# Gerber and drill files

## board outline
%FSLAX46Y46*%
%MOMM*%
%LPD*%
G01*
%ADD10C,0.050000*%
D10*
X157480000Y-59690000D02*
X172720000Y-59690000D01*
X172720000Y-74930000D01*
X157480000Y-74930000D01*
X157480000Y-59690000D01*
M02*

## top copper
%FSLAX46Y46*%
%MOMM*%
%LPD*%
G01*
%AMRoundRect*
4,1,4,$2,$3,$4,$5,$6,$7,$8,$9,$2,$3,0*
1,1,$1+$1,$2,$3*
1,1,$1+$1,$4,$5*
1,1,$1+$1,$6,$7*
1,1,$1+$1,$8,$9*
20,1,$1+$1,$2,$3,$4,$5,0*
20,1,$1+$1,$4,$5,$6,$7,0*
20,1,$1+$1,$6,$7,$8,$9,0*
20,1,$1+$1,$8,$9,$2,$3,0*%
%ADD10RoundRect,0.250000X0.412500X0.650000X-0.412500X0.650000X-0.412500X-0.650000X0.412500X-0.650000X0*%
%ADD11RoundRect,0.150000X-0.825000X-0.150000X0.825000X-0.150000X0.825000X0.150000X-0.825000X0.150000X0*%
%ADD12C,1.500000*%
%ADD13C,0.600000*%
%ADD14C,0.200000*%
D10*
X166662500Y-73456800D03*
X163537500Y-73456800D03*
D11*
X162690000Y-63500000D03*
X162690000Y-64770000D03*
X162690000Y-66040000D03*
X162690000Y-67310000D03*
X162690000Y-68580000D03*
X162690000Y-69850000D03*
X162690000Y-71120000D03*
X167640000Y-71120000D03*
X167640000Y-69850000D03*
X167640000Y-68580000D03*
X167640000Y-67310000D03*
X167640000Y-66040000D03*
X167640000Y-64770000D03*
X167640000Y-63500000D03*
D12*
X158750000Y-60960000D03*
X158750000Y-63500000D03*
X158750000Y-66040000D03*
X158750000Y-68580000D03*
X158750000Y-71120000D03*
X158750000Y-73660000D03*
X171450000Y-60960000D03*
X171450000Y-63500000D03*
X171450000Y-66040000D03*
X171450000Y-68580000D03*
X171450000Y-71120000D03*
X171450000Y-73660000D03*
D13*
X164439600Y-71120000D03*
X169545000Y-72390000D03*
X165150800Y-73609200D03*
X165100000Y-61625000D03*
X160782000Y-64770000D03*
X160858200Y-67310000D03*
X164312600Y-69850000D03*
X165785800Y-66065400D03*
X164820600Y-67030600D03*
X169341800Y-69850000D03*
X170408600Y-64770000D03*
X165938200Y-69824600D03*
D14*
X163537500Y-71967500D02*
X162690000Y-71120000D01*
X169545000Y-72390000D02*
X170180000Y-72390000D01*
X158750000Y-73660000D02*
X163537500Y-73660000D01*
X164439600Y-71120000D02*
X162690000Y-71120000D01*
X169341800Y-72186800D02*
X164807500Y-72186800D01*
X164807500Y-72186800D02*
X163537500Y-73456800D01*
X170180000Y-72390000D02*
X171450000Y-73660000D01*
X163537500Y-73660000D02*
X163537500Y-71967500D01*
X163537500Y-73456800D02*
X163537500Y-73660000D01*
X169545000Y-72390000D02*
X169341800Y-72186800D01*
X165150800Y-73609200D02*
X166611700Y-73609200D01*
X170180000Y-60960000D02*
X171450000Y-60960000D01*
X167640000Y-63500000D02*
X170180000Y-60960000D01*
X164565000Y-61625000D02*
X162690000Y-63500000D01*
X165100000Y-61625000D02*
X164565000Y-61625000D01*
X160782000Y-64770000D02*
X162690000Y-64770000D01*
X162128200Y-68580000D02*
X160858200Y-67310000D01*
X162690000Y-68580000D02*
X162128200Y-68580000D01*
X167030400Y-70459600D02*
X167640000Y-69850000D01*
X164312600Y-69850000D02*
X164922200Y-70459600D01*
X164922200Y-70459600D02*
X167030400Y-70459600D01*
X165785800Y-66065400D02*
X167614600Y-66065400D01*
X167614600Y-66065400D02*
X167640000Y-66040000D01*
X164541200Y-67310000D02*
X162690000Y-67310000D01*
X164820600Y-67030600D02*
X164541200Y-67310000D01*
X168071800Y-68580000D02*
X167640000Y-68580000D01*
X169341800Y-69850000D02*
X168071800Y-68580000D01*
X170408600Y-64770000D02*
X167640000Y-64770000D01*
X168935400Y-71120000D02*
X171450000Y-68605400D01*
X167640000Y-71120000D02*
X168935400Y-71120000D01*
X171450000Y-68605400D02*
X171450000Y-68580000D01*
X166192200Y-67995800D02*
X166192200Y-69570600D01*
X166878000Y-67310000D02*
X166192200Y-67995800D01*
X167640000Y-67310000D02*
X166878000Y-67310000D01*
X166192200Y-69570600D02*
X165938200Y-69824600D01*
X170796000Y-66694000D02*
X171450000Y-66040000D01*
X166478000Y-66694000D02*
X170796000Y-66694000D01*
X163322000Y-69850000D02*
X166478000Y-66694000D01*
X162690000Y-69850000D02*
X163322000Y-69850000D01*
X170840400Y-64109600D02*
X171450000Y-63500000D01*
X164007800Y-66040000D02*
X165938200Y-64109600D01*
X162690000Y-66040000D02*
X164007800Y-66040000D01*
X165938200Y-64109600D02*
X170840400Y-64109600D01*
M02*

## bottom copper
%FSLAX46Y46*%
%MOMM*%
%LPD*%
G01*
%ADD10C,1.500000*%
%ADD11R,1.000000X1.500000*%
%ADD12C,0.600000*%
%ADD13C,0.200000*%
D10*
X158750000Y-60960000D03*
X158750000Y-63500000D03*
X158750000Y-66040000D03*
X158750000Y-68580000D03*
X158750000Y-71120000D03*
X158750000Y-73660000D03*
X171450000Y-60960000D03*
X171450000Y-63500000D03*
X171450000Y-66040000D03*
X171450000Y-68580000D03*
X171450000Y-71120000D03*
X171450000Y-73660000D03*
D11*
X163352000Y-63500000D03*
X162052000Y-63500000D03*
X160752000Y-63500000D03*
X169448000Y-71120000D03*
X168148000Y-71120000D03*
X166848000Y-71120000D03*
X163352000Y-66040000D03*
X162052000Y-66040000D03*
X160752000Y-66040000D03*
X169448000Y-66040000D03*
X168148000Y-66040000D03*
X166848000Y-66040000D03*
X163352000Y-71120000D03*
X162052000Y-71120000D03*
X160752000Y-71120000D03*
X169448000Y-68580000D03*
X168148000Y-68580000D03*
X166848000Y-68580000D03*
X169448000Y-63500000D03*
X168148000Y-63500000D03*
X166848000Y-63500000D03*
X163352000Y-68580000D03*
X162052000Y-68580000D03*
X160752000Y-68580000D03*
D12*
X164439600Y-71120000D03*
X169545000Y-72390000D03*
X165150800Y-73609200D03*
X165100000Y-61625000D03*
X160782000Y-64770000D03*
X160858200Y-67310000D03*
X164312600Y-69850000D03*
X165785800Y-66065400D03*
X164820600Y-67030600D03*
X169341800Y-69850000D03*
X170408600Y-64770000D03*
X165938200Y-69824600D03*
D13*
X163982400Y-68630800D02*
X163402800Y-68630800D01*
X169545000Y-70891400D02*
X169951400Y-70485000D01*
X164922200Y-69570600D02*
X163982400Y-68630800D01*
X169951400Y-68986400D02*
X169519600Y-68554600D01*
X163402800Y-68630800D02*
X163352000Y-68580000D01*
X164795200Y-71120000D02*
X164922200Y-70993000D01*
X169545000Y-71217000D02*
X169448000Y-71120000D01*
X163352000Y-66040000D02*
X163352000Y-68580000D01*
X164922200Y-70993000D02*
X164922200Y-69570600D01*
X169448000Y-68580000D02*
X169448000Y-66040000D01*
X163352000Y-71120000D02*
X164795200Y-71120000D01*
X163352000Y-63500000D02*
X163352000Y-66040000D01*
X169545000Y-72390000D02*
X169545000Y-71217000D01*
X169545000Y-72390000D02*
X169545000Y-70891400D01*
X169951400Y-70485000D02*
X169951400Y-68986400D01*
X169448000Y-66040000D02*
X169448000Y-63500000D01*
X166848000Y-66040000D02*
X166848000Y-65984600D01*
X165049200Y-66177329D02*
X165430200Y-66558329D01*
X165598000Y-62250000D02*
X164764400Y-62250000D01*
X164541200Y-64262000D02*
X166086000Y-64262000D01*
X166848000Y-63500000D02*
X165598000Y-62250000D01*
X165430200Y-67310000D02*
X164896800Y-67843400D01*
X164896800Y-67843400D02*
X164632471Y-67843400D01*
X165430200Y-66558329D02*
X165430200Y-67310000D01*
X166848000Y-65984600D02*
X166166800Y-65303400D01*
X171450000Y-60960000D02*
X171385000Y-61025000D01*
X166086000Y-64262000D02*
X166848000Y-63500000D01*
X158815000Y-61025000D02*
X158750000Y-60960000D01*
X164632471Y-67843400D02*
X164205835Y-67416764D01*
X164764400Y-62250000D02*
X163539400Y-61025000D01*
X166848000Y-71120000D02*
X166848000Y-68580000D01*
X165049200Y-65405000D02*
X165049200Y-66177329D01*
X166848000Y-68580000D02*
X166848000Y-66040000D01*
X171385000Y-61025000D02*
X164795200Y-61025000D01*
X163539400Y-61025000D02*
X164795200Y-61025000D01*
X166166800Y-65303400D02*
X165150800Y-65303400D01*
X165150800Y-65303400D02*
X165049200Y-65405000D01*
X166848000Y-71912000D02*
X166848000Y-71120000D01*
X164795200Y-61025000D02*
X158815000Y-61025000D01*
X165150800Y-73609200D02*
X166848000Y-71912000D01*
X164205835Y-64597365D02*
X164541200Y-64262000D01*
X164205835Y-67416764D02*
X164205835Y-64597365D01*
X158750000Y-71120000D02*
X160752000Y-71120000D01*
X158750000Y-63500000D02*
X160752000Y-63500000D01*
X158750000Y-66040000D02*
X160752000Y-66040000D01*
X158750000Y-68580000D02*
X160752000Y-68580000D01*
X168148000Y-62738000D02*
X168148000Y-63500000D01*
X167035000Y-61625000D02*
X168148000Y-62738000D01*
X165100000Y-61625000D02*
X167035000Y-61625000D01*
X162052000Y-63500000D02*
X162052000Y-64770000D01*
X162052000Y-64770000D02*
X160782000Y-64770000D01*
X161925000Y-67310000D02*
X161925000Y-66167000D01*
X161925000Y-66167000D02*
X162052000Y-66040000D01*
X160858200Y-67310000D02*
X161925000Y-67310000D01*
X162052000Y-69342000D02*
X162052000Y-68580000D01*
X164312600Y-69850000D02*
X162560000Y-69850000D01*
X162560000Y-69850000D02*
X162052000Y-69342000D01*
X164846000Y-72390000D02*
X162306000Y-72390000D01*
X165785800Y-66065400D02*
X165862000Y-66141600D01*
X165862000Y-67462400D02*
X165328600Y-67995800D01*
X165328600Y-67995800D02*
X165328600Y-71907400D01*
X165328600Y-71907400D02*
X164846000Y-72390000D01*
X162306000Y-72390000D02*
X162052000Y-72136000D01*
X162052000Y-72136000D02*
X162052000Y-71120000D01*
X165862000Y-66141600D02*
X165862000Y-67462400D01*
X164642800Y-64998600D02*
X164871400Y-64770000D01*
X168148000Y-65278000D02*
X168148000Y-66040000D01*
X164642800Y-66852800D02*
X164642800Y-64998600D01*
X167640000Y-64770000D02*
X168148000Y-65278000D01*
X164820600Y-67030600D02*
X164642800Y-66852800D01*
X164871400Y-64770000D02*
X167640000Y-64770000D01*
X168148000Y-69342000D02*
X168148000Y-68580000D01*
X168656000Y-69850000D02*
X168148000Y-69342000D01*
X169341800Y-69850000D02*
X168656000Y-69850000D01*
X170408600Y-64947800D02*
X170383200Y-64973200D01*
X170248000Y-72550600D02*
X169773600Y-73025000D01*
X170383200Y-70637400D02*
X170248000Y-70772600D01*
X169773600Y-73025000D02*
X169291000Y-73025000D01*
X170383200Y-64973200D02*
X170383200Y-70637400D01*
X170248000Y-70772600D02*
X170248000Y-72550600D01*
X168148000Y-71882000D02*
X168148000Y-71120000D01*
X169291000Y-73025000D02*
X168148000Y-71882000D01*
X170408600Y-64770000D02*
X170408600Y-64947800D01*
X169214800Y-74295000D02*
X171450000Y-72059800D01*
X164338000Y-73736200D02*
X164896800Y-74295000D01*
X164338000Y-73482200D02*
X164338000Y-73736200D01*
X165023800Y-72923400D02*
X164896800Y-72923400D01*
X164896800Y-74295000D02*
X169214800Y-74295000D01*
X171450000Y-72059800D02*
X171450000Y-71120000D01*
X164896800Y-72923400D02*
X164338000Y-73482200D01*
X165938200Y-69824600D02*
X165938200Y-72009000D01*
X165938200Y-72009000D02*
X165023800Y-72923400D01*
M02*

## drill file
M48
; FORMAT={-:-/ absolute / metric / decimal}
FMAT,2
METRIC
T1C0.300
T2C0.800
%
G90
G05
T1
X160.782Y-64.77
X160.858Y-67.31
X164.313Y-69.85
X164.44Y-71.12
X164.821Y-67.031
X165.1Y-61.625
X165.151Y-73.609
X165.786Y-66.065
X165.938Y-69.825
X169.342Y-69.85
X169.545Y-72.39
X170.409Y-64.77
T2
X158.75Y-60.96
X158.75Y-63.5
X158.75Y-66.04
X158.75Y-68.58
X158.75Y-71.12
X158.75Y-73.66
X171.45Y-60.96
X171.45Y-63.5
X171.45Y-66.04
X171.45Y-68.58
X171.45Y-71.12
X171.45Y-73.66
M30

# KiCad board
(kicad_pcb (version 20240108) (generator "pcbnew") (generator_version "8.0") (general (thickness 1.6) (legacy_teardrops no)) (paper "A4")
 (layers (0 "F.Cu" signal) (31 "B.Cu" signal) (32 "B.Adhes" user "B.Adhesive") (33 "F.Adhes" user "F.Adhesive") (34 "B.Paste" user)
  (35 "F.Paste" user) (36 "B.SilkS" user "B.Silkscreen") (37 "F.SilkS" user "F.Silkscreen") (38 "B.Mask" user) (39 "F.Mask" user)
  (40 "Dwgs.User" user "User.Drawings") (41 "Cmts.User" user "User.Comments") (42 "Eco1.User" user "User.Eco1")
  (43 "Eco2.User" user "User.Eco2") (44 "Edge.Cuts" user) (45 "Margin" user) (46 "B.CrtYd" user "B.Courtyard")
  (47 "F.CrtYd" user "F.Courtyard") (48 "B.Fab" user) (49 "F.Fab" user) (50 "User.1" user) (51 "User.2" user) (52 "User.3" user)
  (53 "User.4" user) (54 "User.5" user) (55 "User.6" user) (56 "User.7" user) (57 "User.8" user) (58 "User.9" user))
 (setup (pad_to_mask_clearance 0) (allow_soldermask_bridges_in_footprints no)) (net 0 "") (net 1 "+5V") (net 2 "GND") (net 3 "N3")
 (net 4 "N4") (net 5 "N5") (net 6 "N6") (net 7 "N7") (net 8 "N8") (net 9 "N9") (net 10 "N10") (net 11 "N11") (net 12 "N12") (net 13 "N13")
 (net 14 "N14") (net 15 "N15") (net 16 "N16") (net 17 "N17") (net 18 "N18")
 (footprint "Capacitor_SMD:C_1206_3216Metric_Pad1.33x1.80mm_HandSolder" (layer "F.Cu") (at 165.1 73.4568 180)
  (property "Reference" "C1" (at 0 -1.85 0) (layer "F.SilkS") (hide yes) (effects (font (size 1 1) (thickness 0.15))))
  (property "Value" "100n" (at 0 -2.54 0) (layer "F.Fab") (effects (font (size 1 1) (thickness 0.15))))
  (pad "1" smd roundrect (at -1.5625 0 180) (size 1.325 1.8) (layers "F.Cu" "F.Paste" "F.Mask") (roundrect_rratio 0.188679) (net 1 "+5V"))
  (pad "2" smd roundrect (at 1.5625 0 180) (size 1.325 1.8) (layers "F.Cu" "F.Paste" "F.Mask") (roundrect_rratio 0.188679) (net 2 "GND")))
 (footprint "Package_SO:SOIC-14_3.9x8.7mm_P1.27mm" (layer "F.Cu") (at 165.165 67.31)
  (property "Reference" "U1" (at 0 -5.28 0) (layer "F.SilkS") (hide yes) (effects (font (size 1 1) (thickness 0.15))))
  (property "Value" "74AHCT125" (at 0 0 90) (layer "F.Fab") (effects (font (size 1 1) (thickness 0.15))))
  (pad "1" smd roundrect (at -2.475 -3.81) (size 1.95 0.6) (layers "F.Cu" "F.Paste" "F.Mask") (roundrect_rratio 0.25) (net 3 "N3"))
  (pad "2" smd roundrect (at -2.475 -2.54) (size 1.95 0.6) (layers "F.Cu" "F.Paste" "F.Mask") (roundrect_rratio 0.25) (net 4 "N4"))
  (pad "3" smd roundrect (at -2.475 -1.27) (size 1.95 0.6) (layers "F.Cu" "F.Paste" "F.Mask") (roundrect_rratio 0.25) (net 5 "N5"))
  (pad "4" smd roundrect (at -2.475 0) (size 1.95 0.6) (layers "F.Cu" "F.Paste" "F.Mask") (roundrect_rratio 0.25) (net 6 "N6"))
  (pad "5" smd roundrect (at -2.475 1.27) (size 1.95 0.6) (layers "F.Cu" "F.Paste" "F.Mask") (roundrect_rratio 0.25) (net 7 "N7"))
  (pad "6" smd roundrect (at -2.475 2.54) (size 1.95 0.6) (layers "F.Cu" "F.Paste" "F.Mask") (roundrect_rratio 0.25) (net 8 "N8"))
  (pad "7" smd roundrect (at -2.475 3.81) (size 1.95 0.6) (layers "F.Cu" "F.Paste" "F.Mask") (roundrect_rratio 0.25) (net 2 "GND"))
  (pad "8" smd roundrect (at 2.475 3.81) (size 1.95 0.6) (layers "F.Cu" "F.Paste" "F.Mask") (roundrect_rratio 0.25) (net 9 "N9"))
  (pad "9" smd roundrect (at 2.475 2.54) (size 1.95 0.6) (layers "F.Cu" "F.Paste" "F.Mask") (roundrect_rratio 0.25) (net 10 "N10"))
  (pad "10" smd roundrect (at 2.475 1.27) (size 1.95 0.6) (layers "F.Cu" "F.Paste" "F.Mask") (roundrect_rratio 0.25) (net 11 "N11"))
  (pad "11" smd roundrect (at 2.475 0) (size 1.95 0.6) (layers "F.Cu" "F.Paste" "F.Mask") (roundrect_rratio 0.25) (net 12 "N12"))
  (pad "12" smd roundrect (at 2.475 -1.27) (size 1.95 0.6) (layers "F.Cu" "F.Paste" "F.Mask") (roundrect_rratio 0.25) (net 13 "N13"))
  (pad "13" smd roundrect (at 2.475 -2.54) (size 1.95 0.6) (layers "F.Cu" "F.Paste" "F.Mask") (roundrect_rratio 0.25) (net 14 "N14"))
  (pad "14" smd roundrect (at 2.475 -3.81) (size 1.95 0.6) (layers "F.Cu" "F.Paste" "F.Mask") (roundrect_rratio 0.25) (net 1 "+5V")))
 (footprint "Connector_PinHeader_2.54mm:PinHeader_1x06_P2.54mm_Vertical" (layer "F.Cu") (at 158.75 60.96)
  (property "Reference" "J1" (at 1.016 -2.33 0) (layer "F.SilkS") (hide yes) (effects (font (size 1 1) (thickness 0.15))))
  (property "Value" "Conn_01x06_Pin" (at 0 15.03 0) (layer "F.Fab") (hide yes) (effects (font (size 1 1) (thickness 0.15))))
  (pad "1" thru_hole circle (at 0 0) (size 1.5 1.5) (drill 0.8) (layers "*.Cu" "*.Mask") (remove_unused_layers no) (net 1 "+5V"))
  (pad "2" thru_hole circle (at 0 2.54) (size 1.5 1.5) (drill 0.8) (layers "*.Cu" "*.Mask") (remove_unused_layers no) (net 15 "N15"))
  (pad "3" thru_hole circle (at 0 5.08) (size 1.5 1.5) (drill 0.8) (layers "*.Cu" "*.Mask") (remove_unused_layers no) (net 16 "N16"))
  (pad "4" thru_hole circle (at 0 7.62) (size 1.5 1.5) (drill 0.8) (layers "*.Cu" "*.Mask") (remove_unused_layers no) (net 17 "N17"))
  (pad "5" thru_hole circle (at 0 10.16) (size 1.5 1.5) (drill 0.8) (layers "*.Cu" "*.Mask") (remove_unused_layers no) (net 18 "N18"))
  (pad "6" thru_hole circle (at 0 12.7) (size 1.5 1.5) (drill 0.8) (layers "*.Cu" "*.Mask") (remove_unused_layers no) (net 2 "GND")))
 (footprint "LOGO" (layer "F.Cu") (at 165.09997 60.628602)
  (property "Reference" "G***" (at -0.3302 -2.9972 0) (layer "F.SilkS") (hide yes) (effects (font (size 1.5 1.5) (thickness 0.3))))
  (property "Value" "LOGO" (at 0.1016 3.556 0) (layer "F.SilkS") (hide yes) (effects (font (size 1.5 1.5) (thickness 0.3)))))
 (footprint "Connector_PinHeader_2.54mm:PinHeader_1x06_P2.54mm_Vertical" (layer "F.Cu") (at 171.45 60.96)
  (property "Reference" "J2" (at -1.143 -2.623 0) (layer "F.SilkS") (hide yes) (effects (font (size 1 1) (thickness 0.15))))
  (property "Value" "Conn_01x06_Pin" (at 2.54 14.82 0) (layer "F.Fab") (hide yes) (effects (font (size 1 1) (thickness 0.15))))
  (pad "1" thru_hole circle (at 0 0 180) (size 1.5 1.5) (drill 0.8) (layers "*.Cu" "*.Mask") (remove_unused_layers no) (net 1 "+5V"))
  (pad "2" thru_hole circle (at 0 2.54 180) (size 1.5 1.5) (drill 0.8) (layers "*.Cu" "*.Mask") (remove_unused_layers no) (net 5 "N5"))
  (pad "3" thru_hole circle (at 0 5.08 180) (size 1.5 1.5) (drill 0.8) (layers "*.Cu" "*.Mask") (remove_unused_layers no) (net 8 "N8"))
  (pad "4" thru_hole circle (at 0 7.62 180) (size 1.5 1.5) (drill 0.8) (layers "*.Cu" "*.Mask") (remove_unused_layers no) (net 9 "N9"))
  (pad "5" thru_hole circle (at 0 10.16 180) (size 1.5 1.5) (drill 0.8) (layers "*.Cu" "*.Mask") (remove_unused_layers no) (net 12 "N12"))
  (pad "6" thru_hole circle (at 0 12.7 180) (size 1.5 1.5) (drill 0.8) (layers "*.Cu" "*.Mask") (remove_unused_layers no) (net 2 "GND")))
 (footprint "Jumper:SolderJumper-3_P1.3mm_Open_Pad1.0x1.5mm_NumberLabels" (layer "B.Cu") (at 162.052 63.5 180)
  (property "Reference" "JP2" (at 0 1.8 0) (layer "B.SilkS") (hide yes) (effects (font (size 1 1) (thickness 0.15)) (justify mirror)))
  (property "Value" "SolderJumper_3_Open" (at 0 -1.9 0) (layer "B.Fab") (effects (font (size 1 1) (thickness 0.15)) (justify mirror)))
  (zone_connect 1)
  (pad "1" smd rect (at -1.3 0 180) (size 1 1.5) (layers "B.Cu" "B.Mask") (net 2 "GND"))
  (pad "2" smd rect (at 0 0 180) (size 1 1.5) (layers "B.Cu" "B.Mask") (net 4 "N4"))
  (pad "3" smd rect (at 1.3 0 180) (size 1 1.5) (layers "B.Cu" "B.Mask") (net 15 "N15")))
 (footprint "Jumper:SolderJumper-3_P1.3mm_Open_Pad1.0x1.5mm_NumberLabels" (layer "B.Cu") (at 168.148 71.12 180)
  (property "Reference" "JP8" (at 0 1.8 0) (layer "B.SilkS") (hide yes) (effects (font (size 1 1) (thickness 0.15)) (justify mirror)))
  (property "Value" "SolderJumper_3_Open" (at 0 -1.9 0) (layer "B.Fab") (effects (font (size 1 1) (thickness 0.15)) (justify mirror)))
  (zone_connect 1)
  (pad "1" smd rect (at -1.3 0 180) (size 1 1.5) (layers "B.Cu" "B.Mask") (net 2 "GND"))
  (pad "2" smd rect (at 0 0 180) (size 1 1.5) (layers "B.Cu" "B.Mask") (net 14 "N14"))
  (pad "3" smd rect (at 1.3 0 180) (size 1 1.5) (layers "B.Cu" "B.Mask") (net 1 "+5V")))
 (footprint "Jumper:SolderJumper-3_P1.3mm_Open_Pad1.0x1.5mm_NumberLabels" (layer "B.Cu") (at 162.052 66.04 180)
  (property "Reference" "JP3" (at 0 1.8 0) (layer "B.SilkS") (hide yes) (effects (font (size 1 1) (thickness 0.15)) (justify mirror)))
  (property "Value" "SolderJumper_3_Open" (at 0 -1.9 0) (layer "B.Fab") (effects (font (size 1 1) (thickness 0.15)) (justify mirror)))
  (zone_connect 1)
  (pad "1" smd rect (at -1.3 0 180) (size 1 1.5) (layers "B.Cu" "B.Mask") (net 2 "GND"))
  (pad "2" smd rect (at 0 0 180) (size 1 1.5) (layers "B.Cu" "B.Mask") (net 7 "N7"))
  (pad "3" smd rect (at 1.3 0 180) (size 1 1.5) (layers "B.Cu" "B.Mask") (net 16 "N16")))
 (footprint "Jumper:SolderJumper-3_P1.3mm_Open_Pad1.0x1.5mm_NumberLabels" (layer "B.Cu") (at 168.148 66.04 180)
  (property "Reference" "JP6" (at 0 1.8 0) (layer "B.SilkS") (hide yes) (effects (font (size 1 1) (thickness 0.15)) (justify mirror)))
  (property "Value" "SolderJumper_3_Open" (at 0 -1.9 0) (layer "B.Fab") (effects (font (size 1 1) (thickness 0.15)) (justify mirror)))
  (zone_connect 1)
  (pad "1" smd rect (at -1.3 0 180) (size 1 1.5) (layers "B.Cu" "B.Mask") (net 2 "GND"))
  (pad "2" smd rect (at 0 0 180) (size 1 1.5) (layers "B.Cu" "B.Mask") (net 6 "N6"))
  (pad "3" smd rect (at 1.3 0 180) (size 1 1.5) (layers "B.Cu" "B.Mask") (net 1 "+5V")))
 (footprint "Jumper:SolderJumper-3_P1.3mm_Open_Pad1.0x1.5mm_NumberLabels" (layer "B.Cu") (at 162.052 71.12 180)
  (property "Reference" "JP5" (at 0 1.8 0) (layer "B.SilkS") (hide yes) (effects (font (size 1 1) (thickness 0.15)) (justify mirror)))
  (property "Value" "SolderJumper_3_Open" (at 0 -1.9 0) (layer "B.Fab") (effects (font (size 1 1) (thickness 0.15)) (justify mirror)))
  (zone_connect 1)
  (pad "1" smd rect (at -1.3 0 180) (size 1 1.5) (layers "B.Cu" "B.Mask") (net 2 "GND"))
  (pad "2" smd rect (at 0 0 180) (size 1 1.5) (layers "B.Cu" "B.Mask") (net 13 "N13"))
  (pad "3" smd rect (at 1.3 0 180) (size 1 1.5) (layers "B.Cu" "B.Mask") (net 18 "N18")))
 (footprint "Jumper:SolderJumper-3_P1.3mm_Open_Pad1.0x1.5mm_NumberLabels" (layer "B.Cu") (at 168.148 68.58 180)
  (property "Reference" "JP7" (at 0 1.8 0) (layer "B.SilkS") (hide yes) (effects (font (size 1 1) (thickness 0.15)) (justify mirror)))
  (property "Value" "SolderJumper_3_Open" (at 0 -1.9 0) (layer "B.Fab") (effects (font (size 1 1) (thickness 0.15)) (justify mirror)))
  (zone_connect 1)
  (pad "1" smd rect (at -1.3 0 180) (size 1 1.5) (layers "B.Cu" "B.Mask") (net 2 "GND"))
  (pad "2" smd rect (at 0 0 180) (size 1 1.5) (layers "B.Cu" "B.Mask") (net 11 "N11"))
  (pad "3" smd rect (at 1.3 0 180) (size 1 1.5) (layers "B.Cu" "B.Mask") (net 1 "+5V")))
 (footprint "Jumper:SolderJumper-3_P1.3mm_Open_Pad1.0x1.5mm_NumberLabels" (layer "B.Cu") (at 168.148 63.5 180)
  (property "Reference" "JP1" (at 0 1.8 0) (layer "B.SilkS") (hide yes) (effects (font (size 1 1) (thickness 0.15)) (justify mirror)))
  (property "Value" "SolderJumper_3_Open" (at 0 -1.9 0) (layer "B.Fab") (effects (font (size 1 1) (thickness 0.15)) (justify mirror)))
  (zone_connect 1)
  (pad "1" smd rect (at -1.3 0 180) (size 1 1.5) (layers "B.Cu" "B.Mask") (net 2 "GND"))
  (pad "2" smd rect (at 0 0 180) (size 1 1.5) (layers "B.Cu" "B.Mask") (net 3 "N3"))
  (pad "3" smd rect (at 1.3 0 180) (size 1 1.5) (layers "B.Cu" "B.Mask") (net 1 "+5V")))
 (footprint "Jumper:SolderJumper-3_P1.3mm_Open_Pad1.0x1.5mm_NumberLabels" (layer "B.Cu") (at 162.052 68.58 180)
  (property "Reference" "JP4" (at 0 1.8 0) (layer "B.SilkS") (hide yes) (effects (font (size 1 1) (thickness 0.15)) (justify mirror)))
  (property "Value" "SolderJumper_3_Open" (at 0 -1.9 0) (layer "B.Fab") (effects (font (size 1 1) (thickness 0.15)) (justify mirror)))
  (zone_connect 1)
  (pad "1" smd rect (at -1.3 0 180) (size 1 1.5) (layers "B.Cu" "B.Mask") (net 2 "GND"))
  (pad "2" smd rect (at 0 0 180) (size 1 1.5) (layers "B.Cu" "B.Mask") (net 10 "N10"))
  (pad "3" smd rect (at 1.3 0 180) (size 1 1.5) (layers "B.Cu" "B.Mask") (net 17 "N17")))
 (gr_rect (start 157.48 59.69) (end 172.72 74.93) (locked yes) (stroke (width 0.05) (type default)) (fill none) (layer "Edge.Cuts"))
 (segment (start 163.5375 71.9675) (end 162.69 71.12) (width 0.2) (layer "F.Cu") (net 2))
 (segment (start 169.545 72.39) (end 170.18 72.39) (width 0.2) (layer "F.Cu") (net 2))
 (segment (start 158.75 73.66) (end 163.5375 73.66) (width 0.2) (layer "F.Cu") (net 2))
 (segment (start 164.4396 71.12) (end 162.69 71.12) (width 0.2) (layer "F.Cu") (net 2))
 (segment (start 169.3418 72.1868) (end 164.8075 72.1868) (width 0.2) (layer "F.Cu") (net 2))
 (segment (start 164.8075 72.1868) (end 163.5375 73.4568) (width 0.2) (layer "F.Cu") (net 2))
 (segment (start 170.18 72.39) (end 171.45 73.66) (width 0.2) (layer "F.Cu") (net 2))
 (segment (start 163.5375 73.66) (end 163.5375 71.9675) (width 0.2) (layer "F.Cu") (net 2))
 (segment (start 163.5375 73.4568) (end 163.5375 73.66) (width 0.2) (layer "F.Cu") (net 2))
 (segment (start 169.545 72.39) (end 169.3418 72.1868) (width 0.2) (layer "F.Cu") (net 2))
 (via (at 164.4396 71.12) (size 0.6) (drill 0.3) (layers "F.Cu" "B.Cu") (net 2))
 (via (at 169.545 72.39) (size 0.6) (drill 0.3) (layers "F.Cu" "B.Cu") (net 2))
 (segment (start 163.9824 68.6308) (end 163.4028 68.6308) (width 0.2) (layer "B.Cu") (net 2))
 (segment (start 169.545 70.8914) (end 169.9514 70.485) (width 0.2) (layer "B.Cu") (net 2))
 (segment (start 164.9222 69.5706) (end 163.9824 68.6308) (width 0.2) (layer "B.Cu") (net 2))
 (segment (start 169.9514 68.9864) (end 169.5196 68.5546) (width 0.2) (layer "B.Cu") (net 2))
 (segment (start 163.4028 68.6308) (end 163.352 68.58) (width 0.2) (layer "B.Cu") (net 2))
 (segment (start 164.7952 71.12) (end 164.9222 70.993) (width 0.2) (layer "B.Cu") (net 2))
 (segment (start 169.545 71.217) (end 169.448 71.12) (width 0.2) (layer "B.Cu") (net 2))
 (segment (start 163.352 66.04) (end 163.352 68.58) (width 0.2) (layer "B.Cu") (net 2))
 (segment (start 164.9222 70.993) (end 164.9222 69.5706) (width 0.2) (layer "B.Cu") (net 2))
 (segment (start 169.448 68.58) (end 169.448 66.04) (width 0.2) (layer "B.Cu") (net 2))
 (segment (start 163.352 71.12) (end 164.7952 71.12) (width 0.2) (layer "B.Cu") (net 2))
 (segment (start 163.352 63.5) (end 163.352 66.04) (width 0.2) (layer "B.Cu") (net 2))
 (segment (start 169.545 72.39) (end 169.545 71.217) (width 0.2) (layer "B.Cu") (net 2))
 (segment (start 169.545 72.39) (end 169.545 70.8914) (width 0.2) (layer "B.Cu") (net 2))
 (segment (start 169.9514 70.485) (end 169.9514 68.9864) (width 0.2) (layer "B.Cu") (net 2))
 (segment (start 169.448 66.04) (end 169.448 63.5) (width 0.2) (layer "B.Cu") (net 2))
 (segment (start 165.1508 73.6092) (end 166.6117 73.6092) (width 0.2) (layer "F.Cu") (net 1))
 (segment (start 170.18 60.96) (end 171.45 60.96) (width 0.2) (layer "F.Cu") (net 1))
 (segment (start 167.64 63.5) (end 170.18 60.96) (width 0.2) (layer "F.Cu") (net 1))
 (via (at 165.1508 73.6092) (size 0.6) (drill 0.3) (layers "F.Cu" "B.Cu") (free yes) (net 1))
 (segment (start 166.848 66.04) (end 166.848 65.9846) (width 0.2) (layer "B.Cu") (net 1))
 (segment (start 165.0492 66.177329) (end 165.4302 66.558329) (width 0.2) (layer "B.Cu") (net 1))
 (segment (start 165.598 62.25) (end 164.7644 62.25) (width 0.2) (layer "B.Cu") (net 1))
 (segment (start 164.5412 64.262) (end 166.086 64.262) (width 0.2) (layer "B.Cu") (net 1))
 (segment (start 166.848 63.5) (end 165.598 62.25) (width 0.2) (layer "B.Cu") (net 1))
 (segment (start 165.4302 67.31) (end 164.8968 67.8434) (width 0.2) (layer "B.Cu") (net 1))
 (segment (start 164.8968 67.8434) (end 164.632471 67.8434) (width 0.2) (layer "B.Cu") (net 1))
 (segment (start 165.4302 66.558329) (end 165.4302 67.31) (width 0.2) (layer "B.Cu") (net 1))
 (segment (start 166.848 65.9846) (end 166.1668 65.3034) (width 0.2) (layer "B.Cu") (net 1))
 (segment (start 171.45 60.96) (end 171.385 61.025) (width 0.2) (layer "B.Cu") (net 1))
 (segment (start 166.086 64.262) (end 166.848 63.5) (width 0.2) (layer "B.Cu") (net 1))
 (segment (start 158.815 61.025) (end 158.75 60.96) (width 0.2) (layer "B.Cu") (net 1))
 (segment (start 164.632471 67.8434) (end 164.205835 67.416764) (width 0.2) (layer "B.Cu") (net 1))
 (segment (start 164.7644 62.25) (end 163.5394 61.025) (width 0.2) (layer "B.Cu") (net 1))
 (segment (start 166.848 71.12) (end 166.848 68.58) (width 0.2) (layer "B.Cu") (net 1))
 (segment (start 165.0492 65.405) (end 165.0492 66.177329) (width 0.2) (layer "B.Cu") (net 1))
 (segment (start 166.848 68.58) (end 166.848 66.04) (width 0.2) (layer "B.Cu") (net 1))
 (segment (start 171.385 61.025) (end 164.7952 61.025) (width 0.2) (layer "B.Cu") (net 1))
 (segment (start 163.5394 61.025) (end 164.7952 61.025) (width 0.2) (layer "B.Cu") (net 1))
 (segment (start 166.1668 65.3034) (end 165.1508 65.3034) (width 0.2) (layer "B.Cu") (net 1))
 (segment (start 165.1508 65.3034) (end 165.0492 65.405) (width 0.2) (layer "B.Cu") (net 1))
 (segment (start 166.848 71.912) (end 166.848 71.12) (width 0.2) (layer "B.Cu") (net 1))
 (segment (start 164.7952 61.025) (end 158.815 61.025) (width 0.2) (layer "B.Cu") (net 1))
 (segment (start 165.1508 73.6092) (end 166.848 71.912) (width 0.2) (layer "B.Cu") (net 1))
 (segment (start 164.205835 64.597365) (end 164.5412 64.262) (width 0.2) (layer "B.Cu") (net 1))
 (segment (start 164.205835 67.416764) (end 164.205835 64.597365) (width 0.2) (layer "B.Cu") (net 1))
 (segment (start 158.75 71.12) (end 160.752 71.12) (width 0.2) (layer "B.Cu") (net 18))
 (segment (start 158.75 63.5) (end 160.752 63.5) (width 0.2) (layer "B.Cu") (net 15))
 (segment (start 158.75 66.04) (end 160.752 66.04) (width 0.2) (layer "B.Cu") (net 16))
 (segment (start 158.75 68.58) (end 160.752 68.58) (width 0.2) (layer "B.Cu") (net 17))
 (segment (start 164.565 61.625) (end 162.69 63.5) (width 0.2) (layer "F.Cu") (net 3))
 (segment (start 165.1 61.625) (end 164.565 61.625) (width 0.2) (layer "F.Cu") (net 3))
 (via (at 165.1 61.625) (size 0.6) (drill 0.3) (layers "F.Cu" "B.Cu") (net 3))
 (segment (start 168.148 62.738) (end 168.148 63.5) (width 0.2) (layer "B.Cu") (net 3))
 (segment (start 167.035 61.625) (end 168.148 62.738) (width 0.2) (layer "B.Cu") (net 3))
 (segment (start 165.1 61.625) (end 167.035 61.625) (width 0.2) (layer "B.Cu") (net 3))
 (segment (start 160.782 64.77) (end 162.69 64.77) (width 0.2) (layer "F.Cu") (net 4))
 (via (at 160.782 64.77) (size 0.6) (drill 0.3) (layers "F.Cu" "B.Cu") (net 4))
 (segment (start 162.052 63.5) (end 162.052 64.77) (width 0.2) (layer "B.Cu") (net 4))
 (segment (start 162.052 64.77) (end 160.782 64.77) (width 0.2) (layer "B.Cu") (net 4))
 (segment (start 162.1282 68.58) (end 160.8582 67.31) (width 0.2) (layer "F.Cu") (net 7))
 (segment (start 162.69 68.58) (end 162.1282 68.58) (width 0.2) (layer "F.Cu") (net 7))
 (via (at 160.8582 67.31) (size 0.6) (drill 0.3) (layers "F.Cu" "B.Cu") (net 7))
 (segment (start 161.925 67.31) (end 161.925 66.167) (width 0.2) (layer "B.Cu") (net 7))
 (segment (start 161.925 66.167) (end 162.052 66.04) (width 0.2) (layer "B.Cu") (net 7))
 (segment (start 160.8582 67.31) (end 161.925 67.31) (width 0.2) (layer "B.Cu") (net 7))
 (segment (start 167.0304 70.4596) (end 167.64 69.85) (width 0.2) (layer "F.Cu") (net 10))
 (segment (start 164.3126 69.85) (end 164.9222 70.4596) (width 0.2) (layer "F.Cu") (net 10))
 (segment (start 164.9222 70.4596) (end 167.0304 70.4596) (width 0.2) (layer "F.Cu") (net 10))
 (via (at 164.3126 69.85) (size 0.6) (drill 0.3) (layers "F.Cu" "B.Cu") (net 10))
 (segment (start 162.052 69.342) (end 162.052 68.58) (width 0.2) (layer "B.Cu") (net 10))
 (segment (start 164.3126 69.85) (end 162.56 69.85) (width 0.2) (layer "B.Cu") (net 10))
 (segment (start 162.56 69.85) (end 162.052 69.342) (width 0.2) (layer "B.Cu") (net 10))
 (segment (start 165.7858 66.0654) (end 167.6146 66.0654) (width 0.2) (layer "F.Cu") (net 13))
 (segment (start 167.6146 66.0654) (end 167.64 66.04) (width 0.2) (layer "F.Cu") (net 13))
 (via (at 165.7858 66.0654) (size 0.6) (drill 0.3) (layers "F.Cu" "B.Cu") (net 13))
 (segment (start 164.846 72.39) (end 162.306 72.39) (width 0.2) (layer "B.Cu") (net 13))
 (segment (start 165.7858 66.0654) (end 165.862 66.1416) (width 0.2) (layer "B.Cu") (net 13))
 (segment (start 165.862 67.4624) (end 165.3286 67.9958) (width 0.2) (layer "B.Cu") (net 13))
 (segment (start 165.3286 67.9958) (end 165.3286 71.9074) (width 0.2) (layer "B.Cu") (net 13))
 (segment (start 165.3286 71.9074) (end 164.846 72.39) (width 0.2) (layer "B.Cu") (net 13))
 (segment (start 162.306 72.39) (end 162.052 72.136) (width 0.2) (layer "B.Cu") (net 13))
 (segment (start 162.052 72.136) (end 162.052 71.12) (width 0.2) (layer "B.Cu") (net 13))
 (segment (start 165.862 66.1416) (end 165.862 67.4624) (width 0.2) (layer "B.Cu") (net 13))
 (segment (start 164.5412 67.31) (end 162.69 67.31) (width 0.2) (layer "F.Cu") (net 6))
 (segment (start 164.8206 67.0306) (end 164.5412 67.31) (width 0.2) (layer "F.Cu") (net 6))
 (via (at 164.8206 67.0306) (size 0.6) (drill 0.3) (layers "F.Cu" "B.Cu") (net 6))
 (segment (start 164.6428 64.9986) (end 164.8714 64.77) (width 0.2) (layer "B.Cu") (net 6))
 (segment (start 168.148 65.278) (end 168.148 66.04) (width 0.2) (layer "B.Cu") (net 6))
 (segment (start 164.6428 66.8528) (end 164.6428 64.9986) (width 0.2) (layer "B.Cu") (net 6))
 (segment (start 167.64 64.77) (end 168.148 65.278) (width 0.2) (layer "B.Cu") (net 6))
 (segment (start 164.8206 67.0306) (end 164.6428 66.8528) (width 0.2) (layer "B.Cu") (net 6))
 (segment (start 164.8714 64.77) (end 167.64 64.77) (width 0.2) (layer "B.Cu") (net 6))
 (segment (start 168.0718 68.58) (end 167.64 68.58) (width 0.2) (layer "F.Cu") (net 11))
 (segment (start 169.3418 69.85) (end 168.0718 68.58) (width 0.2) (layer "F.Cu") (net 11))
 (via (at 169.3418 69.85) (size 0.6) (drill 0.3) (layers "F.Cu" "B.Cu") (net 11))
 (segment (start 168.148 69.342) (end 168.148 68.58) (width 0.2) (layer "B.Cu") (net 11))
 (segment (start 168.656 69.85) (end 168.148 69.342) (width 0.2) (layer "B.Cu") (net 11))
 (segment (start 169.3418 69.85) (end 168.656 69.85) (width 0.2) (layer "B.Cu") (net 11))
 (segment (start 170.4086 64.77) (end 167.64 64.77) (width 0.2) (layer "F.Cu") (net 14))
 (via (at 170.4086 64.77) (size 0.6) (drill 0.3) (layers "F.Cu" "B.Cu") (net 14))
 (segment (start 170.4086 64.9478) (end 170.3832 64.9732) (width 0.2) (layer "B.Cu") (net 14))
 (segment (start 170.248 72.5506) (end 169.7736 73.025) (width 0.2) (layer "B.Cu") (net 14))
 (segment (start 170.3832 70.6374) (end 170.248 70.7726) (width 0.2) (layer "B.Cu") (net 14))
 (segment (start 169.7736 73.025) (end 169.291 73.025) (width 0.2) (layer "B.Cu") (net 14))
 (segment (start 170.3832 64.9732) (end 170.3832 70.6374) (width 0.2) (layer "B.Cu") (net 14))
 (segment (start 170.248 70.7726) (end 170.248 72.5506) (width 0.2) (layer "B.Cu") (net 14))
 (segment (start 168.148 71.882) (end 168.148 71.12) (width 0.2) (layer "B.Cu") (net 14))
 (segment (start 169.291 73.025) (end 168.148 71.882) (width 0.2) (layer "B.Cu") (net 14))
 (segment (start 170.4086 64.77) (end 170.4086 64.9478) (width 0.2) (layer "B.Cu") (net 14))
 (segment (start 168.9354 71.12) (end 171.45 68.6054) (width 0.2) (layer "F.Cu") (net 9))
 (segment (start 167.64 71.12) (end 168.9354 71.12) (width 0.2) (layer "F.Cu") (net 9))
 (segment (start 171.45 68.6054) (end 171.45 68.58) (width 0.2) (layer "F.Cu") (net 9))
 (segment (start 166.1922 67.9958) (end 166.1922 69.5706) (width 0.2) (layer "F.Cu") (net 12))
 (segment (start 166.878 67.31) (end 166.1922 67.9958) (width 0.2) (layer "F.Cu") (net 12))
 (segment (start 167.64 67.31) (end 166.878 67.31) (width 0.2) (layer "F.Cu") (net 12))
 (segment (start 166.1922 69.5706) (end 165.9382 69.8246) (width 0.2) (layer "F.Cu") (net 12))
 (via (at 165.9382 69.8246) (size 0.6) (drill 0.3) (layers "F.Cu" "B.Cu") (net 12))
 (segment (start 169.2148 74.295) (end 171.45 72.0598) (width 0.2) (layer "B.Cu") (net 12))
 (segment (start 164.338 73.7362) (end 164.8968 74.295) (width 0.2) (layer "B.Cu") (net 12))
 (segment (start 164.338 73.4822) (end 164.338 73.7362) (width 0.2) (layer "B.Cu") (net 12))
 (segment (start 165.0238 72.9234) (end 164.8968 72.9234) (width 0.2) (layer "B.Cu") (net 12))
 (segment (start 164.8968 74.295) (end 169.2148 74.295) (width 0.2) (layer "B.Cu") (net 12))
 (segment (start 171.45 72.0598) (end 171.45 71.12) (width 0.2) (layer "B.Cu") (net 12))
 (segment (start 164.8968 72.9234) (end 164.338 73.4822) (width 0.2) (layer "B.Cu") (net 12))
 (segment (start 165.9382 69.8246) (end 165.9382 72.009) (width 0.2) (layer "B.Cu") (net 12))
 (segment (start 165.9382 72.009) (end 165.0238 72.9234) (width 0.2) (layer "B.Cu") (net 12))
 (segment (start 170.796 66.694) (end 171.45 66.04) (width 0.2) (layer "F.Cu") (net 8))
 (segment (start 166.478 66.694) (end 170.796 66.694) (width 0.2) (layer "F.Cu") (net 8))
 (segment (start 163.322 69.85) (end 166.478 66.694) (width 0.2) (layer "F.Cu") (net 8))
 (segment (start 162.69 69.85) (end 163.322 69.85) (width 0.2) (layer "F.Cu") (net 8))
 (segment (start 170.8404 64.1096) (end 171.45 63.5) (width 0.2) (layer "F.Cu") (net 5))
 (segment (start 164.0078 66.04) (end 165.9382 64.1096) (width 0.2) (layer "F.Cu") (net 5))
 (segment (start 162.69 66.04) (end 164.0078 66.04) (width 0.2) (layer "F.Cu") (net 5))
 (segment (start 165.9382 64.1096) (end 170.8404 64.1096) (width 0.2) (layer "F.Cu") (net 5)))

